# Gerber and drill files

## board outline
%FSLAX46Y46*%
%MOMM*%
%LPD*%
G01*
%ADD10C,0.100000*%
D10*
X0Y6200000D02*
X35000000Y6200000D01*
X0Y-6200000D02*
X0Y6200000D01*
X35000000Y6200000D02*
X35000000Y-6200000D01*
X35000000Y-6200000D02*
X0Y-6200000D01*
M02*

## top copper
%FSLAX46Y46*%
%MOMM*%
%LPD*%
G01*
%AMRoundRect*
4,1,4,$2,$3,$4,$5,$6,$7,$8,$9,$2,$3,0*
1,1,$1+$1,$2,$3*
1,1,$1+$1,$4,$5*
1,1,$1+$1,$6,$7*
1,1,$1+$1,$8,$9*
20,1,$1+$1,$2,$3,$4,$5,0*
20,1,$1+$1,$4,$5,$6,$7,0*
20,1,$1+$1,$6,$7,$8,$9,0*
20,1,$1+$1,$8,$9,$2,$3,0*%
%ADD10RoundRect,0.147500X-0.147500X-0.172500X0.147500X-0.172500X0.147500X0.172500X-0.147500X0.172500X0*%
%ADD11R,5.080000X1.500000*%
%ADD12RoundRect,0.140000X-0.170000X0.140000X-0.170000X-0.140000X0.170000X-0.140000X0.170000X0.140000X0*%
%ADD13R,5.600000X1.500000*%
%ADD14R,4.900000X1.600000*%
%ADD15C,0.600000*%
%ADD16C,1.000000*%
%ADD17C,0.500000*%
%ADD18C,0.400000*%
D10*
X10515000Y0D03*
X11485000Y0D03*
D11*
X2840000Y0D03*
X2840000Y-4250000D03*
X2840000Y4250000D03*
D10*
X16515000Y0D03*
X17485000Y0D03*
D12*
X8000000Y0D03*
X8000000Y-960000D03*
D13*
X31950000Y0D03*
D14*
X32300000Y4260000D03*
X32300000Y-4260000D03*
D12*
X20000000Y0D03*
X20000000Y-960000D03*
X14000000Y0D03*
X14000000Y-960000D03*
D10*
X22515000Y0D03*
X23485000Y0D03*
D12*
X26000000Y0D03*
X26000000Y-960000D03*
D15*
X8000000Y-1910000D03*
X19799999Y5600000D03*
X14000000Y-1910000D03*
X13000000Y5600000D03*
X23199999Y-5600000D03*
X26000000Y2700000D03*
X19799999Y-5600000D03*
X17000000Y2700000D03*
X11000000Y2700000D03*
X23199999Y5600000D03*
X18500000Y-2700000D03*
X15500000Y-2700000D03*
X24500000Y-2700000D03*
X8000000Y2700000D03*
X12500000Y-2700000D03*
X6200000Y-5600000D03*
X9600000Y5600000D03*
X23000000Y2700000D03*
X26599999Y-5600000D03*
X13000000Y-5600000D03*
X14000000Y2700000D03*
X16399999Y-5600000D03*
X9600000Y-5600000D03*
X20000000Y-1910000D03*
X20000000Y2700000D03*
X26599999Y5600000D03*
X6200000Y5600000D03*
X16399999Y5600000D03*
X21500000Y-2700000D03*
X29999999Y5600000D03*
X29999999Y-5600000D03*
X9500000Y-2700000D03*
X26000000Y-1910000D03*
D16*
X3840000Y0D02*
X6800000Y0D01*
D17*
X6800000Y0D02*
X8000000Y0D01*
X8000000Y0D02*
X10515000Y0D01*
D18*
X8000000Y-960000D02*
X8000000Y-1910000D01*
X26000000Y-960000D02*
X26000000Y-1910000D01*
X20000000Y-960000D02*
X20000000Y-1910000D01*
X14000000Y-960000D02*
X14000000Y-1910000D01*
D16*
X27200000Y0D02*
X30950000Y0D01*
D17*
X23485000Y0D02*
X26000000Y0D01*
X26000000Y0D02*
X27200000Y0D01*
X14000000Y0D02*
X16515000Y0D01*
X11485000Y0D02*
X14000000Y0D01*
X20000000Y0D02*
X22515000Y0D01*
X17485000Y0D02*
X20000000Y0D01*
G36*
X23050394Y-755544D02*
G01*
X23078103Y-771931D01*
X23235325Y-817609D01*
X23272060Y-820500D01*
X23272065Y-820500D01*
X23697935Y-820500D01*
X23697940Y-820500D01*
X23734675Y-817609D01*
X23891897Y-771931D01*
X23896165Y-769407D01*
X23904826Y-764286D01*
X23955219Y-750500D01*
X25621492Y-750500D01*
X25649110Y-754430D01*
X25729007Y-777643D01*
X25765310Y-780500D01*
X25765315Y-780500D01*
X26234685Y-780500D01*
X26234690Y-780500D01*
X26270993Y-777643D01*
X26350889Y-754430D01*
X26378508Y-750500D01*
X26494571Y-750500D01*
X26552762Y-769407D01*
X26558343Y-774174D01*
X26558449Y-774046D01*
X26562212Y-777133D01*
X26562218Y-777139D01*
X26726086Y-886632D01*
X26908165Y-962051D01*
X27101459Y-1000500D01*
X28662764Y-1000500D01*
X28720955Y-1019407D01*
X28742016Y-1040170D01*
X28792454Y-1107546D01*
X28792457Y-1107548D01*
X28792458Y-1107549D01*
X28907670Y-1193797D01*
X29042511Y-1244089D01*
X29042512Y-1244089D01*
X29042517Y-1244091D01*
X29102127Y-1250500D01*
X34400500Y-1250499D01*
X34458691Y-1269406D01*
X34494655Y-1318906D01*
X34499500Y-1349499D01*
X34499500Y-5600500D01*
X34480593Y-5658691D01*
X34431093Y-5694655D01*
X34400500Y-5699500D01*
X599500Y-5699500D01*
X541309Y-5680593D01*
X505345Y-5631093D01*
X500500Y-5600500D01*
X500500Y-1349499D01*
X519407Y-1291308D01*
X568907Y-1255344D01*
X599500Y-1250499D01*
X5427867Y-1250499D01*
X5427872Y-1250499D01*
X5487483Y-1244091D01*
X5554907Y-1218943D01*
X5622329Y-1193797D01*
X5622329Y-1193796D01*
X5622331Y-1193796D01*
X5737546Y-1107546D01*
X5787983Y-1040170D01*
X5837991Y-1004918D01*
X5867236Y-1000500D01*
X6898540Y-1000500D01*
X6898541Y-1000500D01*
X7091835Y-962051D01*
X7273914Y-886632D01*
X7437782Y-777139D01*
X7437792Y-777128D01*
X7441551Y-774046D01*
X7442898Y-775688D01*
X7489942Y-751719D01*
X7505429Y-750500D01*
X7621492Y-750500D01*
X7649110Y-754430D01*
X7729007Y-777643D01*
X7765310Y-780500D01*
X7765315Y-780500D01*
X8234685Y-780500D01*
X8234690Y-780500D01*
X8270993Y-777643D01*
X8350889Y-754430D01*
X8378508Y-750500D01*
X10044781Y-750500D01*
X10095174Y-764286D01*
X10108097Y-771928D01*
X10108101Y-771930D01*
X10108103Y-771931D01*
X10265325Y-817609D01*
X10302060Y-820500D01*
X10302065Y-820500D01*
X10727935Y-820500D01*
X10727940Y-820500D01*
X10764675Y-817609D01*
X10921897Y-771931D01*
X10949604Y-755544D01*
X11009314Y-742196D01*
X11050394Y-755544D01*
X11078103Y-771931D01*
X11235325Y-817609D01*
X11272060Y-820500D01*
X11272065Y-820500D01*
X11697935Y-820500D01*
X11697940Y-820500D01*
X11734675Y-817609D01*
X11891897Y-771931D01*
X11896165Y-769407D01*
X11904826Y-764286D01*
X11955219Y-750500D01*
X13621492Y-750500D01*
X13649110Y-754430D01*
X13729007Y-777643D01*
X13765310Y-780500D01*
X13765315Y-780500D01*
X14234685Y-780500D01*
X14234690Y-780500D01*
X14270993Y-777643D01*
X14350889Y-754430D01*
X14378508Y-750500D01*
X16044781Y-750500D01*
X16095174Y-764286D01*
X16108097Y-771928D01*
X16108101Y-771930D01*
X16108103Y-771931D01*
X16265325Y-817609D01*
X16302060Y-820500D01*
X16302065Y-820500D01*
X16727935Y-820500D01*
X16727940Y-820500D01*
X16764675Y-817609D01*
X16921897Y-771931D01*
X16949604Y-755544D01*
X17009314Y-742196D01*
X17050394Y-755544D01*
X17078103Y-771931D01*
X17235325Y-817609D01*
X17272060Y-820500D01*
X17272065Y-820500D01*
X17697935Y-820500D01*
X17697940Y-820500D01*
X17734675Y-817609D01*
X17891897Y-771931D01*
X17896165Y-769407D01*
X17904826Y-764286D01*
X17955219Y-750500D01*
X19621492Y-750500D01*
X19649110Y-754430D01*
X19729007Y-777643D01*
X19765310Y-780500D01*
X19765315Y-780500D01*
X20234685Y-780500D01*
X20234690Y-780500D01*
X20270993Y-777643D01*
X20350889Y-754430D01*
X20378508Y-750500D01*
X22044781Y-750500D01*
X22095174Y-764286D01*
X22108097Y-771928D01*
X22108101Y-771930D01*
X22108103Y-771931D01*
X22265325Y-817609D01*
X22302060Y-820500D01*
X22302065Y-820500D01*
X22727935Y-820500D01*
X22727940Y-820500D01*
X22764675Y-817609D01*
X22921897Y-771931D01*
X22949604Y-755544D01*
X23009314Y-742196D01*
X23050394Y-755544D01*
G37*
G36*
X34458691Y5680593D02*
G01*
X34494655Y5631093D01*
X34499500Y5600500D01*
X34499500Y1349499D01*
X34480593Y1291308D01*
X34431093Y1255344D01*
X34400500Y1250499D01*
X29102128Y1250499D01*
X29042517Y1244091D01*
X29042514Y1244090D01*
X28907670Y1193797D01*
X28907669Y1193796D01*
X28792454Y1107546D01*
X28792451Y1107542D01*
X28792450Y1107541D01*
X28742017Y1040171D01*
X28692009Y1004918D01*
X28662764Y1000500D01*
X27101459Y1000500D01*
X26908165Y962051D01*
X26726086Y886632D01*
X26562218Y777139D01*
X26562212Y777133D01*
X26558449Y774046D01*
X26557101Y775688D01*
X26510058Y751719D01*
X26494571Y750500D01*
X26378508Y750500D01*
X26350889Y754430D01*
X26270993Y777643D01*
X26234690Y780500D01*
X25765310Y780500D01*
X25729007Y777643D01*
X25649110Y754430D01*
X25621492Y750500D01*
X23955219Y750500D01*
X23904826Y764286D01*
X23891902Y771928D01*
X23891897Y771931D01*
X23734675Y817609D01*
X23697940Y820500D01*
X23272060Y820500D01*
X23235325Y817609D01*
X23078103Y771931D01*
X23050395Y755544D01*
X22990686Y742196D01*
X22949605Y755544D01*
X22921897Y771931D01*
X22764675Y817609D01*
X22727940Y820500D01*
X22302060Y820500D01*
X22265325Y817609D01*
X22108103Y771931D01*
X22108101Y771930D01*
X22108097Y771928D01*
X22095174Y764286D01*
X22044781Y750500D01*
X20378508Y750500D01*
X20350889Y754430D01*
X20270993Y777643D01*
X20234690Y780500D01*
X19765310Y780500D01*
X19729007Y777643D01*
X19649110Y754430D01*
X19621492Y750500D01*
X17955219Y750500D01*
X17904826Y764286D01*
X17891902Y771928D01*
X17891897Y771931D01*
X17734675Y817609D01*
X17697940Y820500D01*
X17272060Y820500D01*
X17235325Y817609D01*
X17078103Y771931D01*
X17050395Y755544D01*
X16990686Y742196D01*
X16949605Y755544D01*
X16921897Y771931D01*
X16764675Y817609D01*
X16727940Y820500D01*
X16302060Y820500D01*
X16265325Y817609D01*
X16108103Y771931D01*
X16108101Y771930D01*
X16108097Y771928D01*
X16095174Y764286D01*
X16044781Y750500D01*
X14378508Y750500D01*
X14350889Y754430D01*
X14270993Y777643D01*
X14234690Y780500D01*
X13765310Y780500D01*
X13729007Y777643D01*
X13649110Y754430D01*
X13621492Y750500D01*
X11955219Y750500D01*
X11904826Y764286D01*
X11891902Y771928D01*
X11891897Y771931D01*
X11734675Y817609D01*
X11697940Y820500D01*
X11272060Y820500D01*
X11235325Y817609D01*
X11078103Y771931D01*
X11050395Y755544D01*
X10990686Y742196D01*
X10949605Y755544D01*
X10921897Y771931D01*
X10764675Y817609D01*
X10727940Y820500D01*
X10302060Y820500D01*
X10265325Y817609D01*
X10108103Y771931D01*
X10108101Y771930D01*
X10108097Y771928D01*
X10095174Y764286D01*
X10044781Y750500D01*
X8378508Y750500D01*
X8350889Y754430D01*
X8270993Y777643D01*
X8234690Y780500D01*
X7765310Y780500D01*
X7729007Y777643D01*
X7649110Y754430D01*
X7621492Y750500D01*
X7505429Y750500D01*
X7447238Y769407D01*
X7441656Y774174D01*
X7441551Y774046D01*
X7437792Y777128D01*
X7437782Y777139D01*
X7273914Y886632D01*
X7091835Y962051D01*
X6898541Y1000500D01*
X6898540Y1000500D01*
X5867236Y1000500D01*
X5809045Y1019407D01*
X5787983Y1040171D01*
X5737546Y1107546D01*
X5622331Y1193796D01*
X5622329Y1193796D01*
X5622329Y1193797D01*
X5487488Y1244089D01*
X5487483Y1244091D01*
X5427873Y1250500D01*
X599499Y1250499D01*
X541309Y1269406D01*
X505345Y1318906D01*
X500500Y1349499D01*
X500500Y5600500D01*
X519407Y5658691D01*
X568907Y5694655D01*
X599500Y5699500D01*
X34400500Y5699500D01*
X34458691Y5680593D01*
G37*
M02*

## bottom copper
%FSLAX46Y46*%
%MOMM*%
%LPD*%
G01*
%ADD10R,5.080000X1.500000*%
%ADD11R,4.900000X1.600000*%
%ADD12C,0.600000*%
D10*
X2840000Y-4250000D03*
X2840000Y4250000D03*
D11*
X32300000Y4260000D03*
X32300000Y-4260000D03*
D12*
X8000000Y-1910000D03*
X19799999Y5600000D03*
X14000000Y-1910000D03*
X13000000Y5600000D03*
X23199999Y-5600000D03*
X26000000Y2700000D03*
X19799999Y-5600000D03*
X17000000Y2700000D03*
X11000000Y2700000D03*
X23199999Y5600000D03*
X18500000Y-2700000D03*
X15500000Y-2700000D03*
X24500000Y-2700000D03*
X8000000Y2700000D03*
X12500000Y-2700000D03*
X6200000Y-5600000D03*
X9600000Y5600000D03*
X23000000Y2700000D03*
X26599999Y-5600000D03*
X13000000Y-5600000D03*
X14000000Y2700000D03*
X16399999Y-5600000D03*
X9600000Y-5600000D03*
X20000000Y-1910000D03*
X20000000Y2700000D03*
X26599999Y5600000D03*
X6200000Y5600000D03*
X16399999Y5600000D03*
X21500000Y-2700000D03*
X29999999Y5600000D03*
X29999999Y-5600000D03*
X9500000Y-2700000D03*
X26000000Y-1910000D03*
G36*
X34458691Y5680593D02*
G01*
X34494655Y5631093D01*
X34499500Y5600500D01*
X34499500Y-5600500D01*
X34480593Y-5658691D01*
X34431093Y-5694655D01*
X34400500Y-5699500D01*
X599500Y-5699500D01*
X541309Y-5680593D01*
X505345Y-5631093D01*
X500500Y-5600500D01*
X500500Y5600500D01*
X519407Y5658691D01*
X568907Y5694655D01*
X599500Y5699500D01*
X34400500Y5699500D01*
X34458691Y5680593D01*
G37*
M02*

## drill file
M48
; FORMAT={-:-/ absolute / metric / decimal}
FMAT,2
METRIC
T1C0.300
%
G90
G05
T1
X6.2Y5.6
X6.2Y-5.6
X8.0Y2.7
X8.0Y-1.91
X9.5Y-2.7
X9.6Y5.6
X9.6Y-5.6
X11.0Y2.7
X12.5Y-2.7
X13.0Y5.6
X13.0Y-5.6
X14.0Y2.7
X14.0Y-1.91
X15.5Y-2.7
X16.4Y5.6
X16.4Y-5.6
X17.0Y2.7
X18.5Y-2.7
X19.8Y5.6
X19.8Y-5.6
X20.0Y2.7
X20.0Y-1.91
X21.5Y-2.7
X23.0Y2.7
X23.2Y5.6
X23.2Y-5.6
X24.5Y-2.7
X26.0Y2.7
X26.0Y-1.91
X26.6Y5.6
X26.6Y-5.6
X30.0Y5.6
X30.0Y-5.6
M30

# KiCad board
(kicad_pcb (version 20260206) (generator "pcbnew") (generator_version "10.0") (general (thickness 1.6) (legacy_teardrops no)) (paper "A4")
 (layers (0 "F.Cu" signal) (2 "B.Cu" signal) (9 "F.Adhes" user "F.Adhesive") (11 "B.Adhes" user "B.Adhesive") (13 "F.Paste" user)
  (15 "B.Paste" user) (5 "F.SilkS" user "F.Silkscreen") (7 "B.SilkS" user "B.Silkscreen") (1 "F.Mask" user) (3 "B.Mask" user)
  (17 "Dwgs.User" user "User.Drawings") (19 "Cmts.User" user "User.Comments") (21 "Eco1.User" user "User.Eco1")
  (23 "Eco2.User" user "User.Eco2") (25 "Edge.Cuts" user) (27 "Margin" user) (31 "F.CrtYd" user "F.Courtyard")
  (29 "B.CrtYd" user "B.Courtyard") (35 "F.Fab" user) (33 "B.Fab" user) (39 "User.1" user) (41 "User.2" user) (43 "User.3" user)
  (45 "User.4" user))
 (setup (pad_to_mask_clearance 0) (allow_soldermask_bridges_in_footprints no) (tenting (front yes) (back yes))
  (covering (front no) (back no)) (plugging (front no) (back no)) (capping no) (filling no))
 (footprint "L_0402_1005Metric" (layer "F.Cu") (at 11 0)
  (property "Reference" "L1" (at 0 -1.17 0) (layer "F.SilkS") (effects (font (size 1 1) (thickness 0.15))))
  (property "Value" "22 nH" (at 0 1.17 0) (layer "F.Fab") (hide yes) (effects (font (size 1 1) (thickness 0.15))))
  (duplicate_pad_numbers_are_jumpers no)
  (pad "1" smd roundrect (at -0.485 0) (size 0.59 0.64) (layers "F.Cu" "F.Mask" "F.Paste") (roundrect_rratio 0.25) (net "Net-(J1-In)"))
  (pad "2" smd roundrect (at 0.485 0) (size 0.59 0.64) (layers "F.Cu" "F.Mask" "F.Paste") (roundrect_rratio 0.25) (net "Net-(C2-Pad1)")))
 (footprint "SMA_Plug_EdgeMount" (layer "F.Cu") (at 2.84 0 180)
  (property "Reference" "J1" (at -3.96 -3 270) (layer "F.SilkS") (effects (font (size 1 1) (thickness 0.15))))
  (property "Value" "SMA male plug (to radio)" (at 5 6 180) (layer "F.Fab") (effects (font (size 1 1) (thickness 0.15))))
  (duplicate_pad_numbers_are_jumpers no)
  (pad "1" smd rect (at 0 0 270) (size 1.5 5.08) (layers "F.Cu" "F.Mask" "F.Paste") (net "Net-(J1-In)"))
  (pad "2" smd rect (at 0 -4.25 270) (size 1.5 5.08) (layers "F.Cu" "F.Mask" "F.Paste") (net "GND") (zone_connect 2))
  (pad "2" smd rect (at 0 -4.25 270) (size 1.5 5.08) (layers "B.Cu" "B.Mask" "B.Paste") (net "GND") (zone_connect 2))
  (pad "2" smd rect (at 0 4.25 270) (size 1.5 5.08) (layers "F.Cu" "F.Mask" "F.Paste") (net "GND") (zone_connect 2))
  (pad "2" smd rect (at 0 4.25 270) (size 1.5 5.08) (layers "B.Cu" "B.Mask" "B.Paste") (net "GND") (zone_connect 2)))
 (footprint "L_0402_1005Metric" (layer "F.Cu") (at 17 0)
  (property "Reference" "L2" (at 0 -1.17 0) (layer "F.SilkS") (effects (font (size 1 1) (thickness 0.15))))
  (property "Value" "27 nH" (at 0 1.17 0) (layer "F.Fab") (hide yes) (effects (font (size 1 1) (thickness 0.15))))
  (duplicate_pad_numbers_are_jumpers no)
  (pad "1" smd roundrect (at -0.485 0) (size 0.59 0.64) (layers "F.Cu" "F.Mask" "F.Paste") (roundrect_rratio 0.25) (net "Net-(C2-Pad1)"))
  (pad "2" smd roundrect (at 0.485 0) (size 0.59 0.64) (layers "F.Cu" "F.Mask" "F.Paste") (roundrect_rratio 0.25) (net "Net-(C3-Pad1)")))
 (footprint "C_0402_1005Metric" (layer "F.Cu") (at 8 0.48 -90)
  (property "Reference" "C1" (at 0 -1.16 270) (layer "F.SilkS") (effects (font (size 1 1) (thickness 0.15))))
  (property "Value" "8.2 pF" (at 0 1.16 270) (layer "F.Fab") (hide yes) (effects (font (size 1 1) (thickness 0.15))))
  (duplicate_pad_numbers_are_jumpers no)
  (pad "1" smd roundrect (at -0.48 0 270) (size 0.56 0.62) (layers "F.Cu" "F.Mask" "F.Paste") (roundrect_rratio 0.25) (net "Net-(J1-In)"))
  (pad "2" smd roundrect (at 0.48 0 270) (size 0.56 0.62) (layers "F.Cu" "F.Mask" "F.Paste") (roundrect_rratio 0.25) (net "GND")
   (zone_connect 2)))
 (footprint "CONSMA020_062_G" (layer "F.Cu") (at 34.75 0)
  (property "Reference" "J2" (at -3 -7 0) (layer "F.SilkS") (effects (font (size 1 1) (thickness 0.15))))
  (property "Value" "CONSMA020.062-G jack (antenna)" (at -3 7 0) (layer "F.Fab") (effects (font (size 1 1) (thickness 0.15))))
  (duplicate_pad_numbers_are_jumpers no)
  (pad "1" smd rect (at -2.8 0) (size 5.6 1.5) (layers "F.Cu" "F.Mask" "F.Paste") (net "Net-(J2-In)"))
  (pad "2" smd rect (at -2.45 -4.26) (size 4.9 1.6) (layers "F.Cu" "F.Mask" "F.Paste") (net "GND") (zone_connect 2))
  (pad "2" smd rect (at -2.45 -4.26) (size 4.9 1.6) (layers "B.Cu" "B.Mask" "B.Paste") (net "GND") (zone_connect 2))
  (pad "2" smd rect (at -2.45 4.26) (size 4.9 1.6) (layers "F.Cu" "F.Mask" "F.Paste") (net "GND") (zone_connect 2))
  (pad "2" smd rect (at -2.45 4.26) (size 4.9 1.6) (layers "B.Cu" "B.Mask" "B.Paste") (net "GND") (zone_connect 2)))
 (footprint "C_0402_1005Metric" (layer "F.Cu") (at 20 0.48 -90)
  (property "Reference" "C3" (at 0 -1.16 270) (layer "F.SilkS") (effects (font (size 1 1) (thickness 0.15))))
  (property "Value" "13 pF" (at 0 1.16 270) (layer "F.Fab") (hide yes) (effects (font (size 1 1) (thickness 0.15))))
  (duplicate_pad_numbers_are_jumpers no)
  (pad "1" smd roundrect (at -0.48 0 270) (size 0.56 0.62) (layers "F.Cu" "F.Mask" "F.Paste") (roundrect_rratio 0.25) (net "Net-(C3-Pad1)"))
  (pad "2" smd roundrect (at 0.48 0 270) (size 0.56 0.62) (layers "F.Cu" "F.Mask" "F.Paste") (roundrect_rratio 0.25) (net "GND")
   (zone_connect 2)))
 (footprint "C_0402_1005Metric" (layer "F.Cu") (at 14 0.48 -90)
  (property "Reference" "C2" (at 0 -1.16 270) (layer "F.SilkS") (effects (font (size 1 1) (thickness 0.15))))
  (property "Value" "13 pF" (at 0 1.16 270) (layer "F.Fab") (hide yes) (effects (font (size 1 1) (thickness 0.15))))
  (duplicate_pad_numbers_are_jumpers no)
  (pad "1" smd roundrect (at -0.48 0 270) (size 0.56 0.62) (layers "F.Cu" "F.Mask" "F.Paste") (roundrect_rratio 0.25) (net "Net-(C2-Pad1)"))
  (pad "2" smd roundrect (at 0.48 0 270) (size 0.56 0.62) (layers "F.Cu" "F.Mask" "F.Paste") (roundrect_rratio 0.25) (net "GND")
   (zone_connect 2)))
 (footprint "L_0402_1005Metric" (layer "F.Cu") (at 23 0)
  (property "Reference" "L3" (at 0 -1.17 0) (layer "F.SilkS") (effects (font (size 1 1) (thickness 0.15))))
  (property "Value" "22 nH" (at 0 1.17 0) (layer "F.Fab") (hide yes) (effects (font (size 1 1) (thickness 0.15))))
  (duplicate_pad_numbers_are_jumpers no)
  (pad "1" smd roundrect (at -0.485 0) (size 0.59 0.64) (layers "F.Cu" "F.Mask" "F.Paste") (roundrect_rratio 0.25) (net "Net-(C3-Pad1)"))
  (pad "2" smd roundrect (at 0.485 0) (size 0.59 0.64) (layers "F.Cu" "F.Mask" "F.Paste") (roundrect_rratio 0.25) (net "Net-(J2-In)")))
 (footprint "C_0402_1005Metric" (layer "F.Cu") (at 26 0.48 -90)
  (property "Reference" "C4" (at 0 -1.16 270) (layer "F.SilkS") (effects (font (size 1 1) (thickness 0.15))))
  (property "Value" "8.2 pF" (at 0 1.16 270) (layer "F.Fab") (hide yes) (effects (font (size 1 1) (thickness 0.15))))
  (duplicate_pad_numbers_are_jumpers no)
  (pad "1" smd roundrect (at -0.48 0 270) (size 0.56 0.62) (layers "F.Cu" "F.Mask" "F.Paste") (roundrect_rratio 0.25) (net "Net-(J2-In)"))
  (pad "2" smd roundrect (at 0.48 0 270) (size 0.56 0.62) (layers "F.Cu" "F.Mask" "F.Paste") (roundrect_rratio 0.25) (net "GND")
   (zone_connect 2)))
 (gr_line (start 0 -6.2) (end 35 -6.2) (stroke (width 0.1) (type default)) (layer "Edge.Cuts"))
 (gr_line (start 0 6.2) (end 0 -6.2) (stroke (width 0.1) (type default)) (layer "Edge.Cuts"))
 (gr_line (start 35 -6.2) (end 35 6.2) (stroke (width 0.1) (type default)) (layer "Edge.Cuts"))
 (gr_line (start 35 6.2) (end 0 6.2) (stroke (width 0.1) (type default)) (layer "Edge.Cuts"))
 (segment (start 3.84 0) (end 6.8 0) (width 1) (layer "F.Cu") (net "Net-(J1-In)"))
 (segment (start 6.8 0) (end 8 0) (width 0.5) (layer "F.Cu") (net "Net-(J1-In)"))
 (segment (start 8 0) (end 10.515 0) (width 0.5) (layer "F.Cu") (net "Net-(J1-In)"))
 (segment (start 8 0.96) (end 8 1.91) (width 0.4) (layer "F.Cu") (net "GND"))
 (segment (start 26 0.96) (end 26 1.91) (width 0.4) (layer "F.Cu") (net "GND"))
 (segment (start 20 0.96) (end 20 1.91) (width 0.4) (layer "F.Cu") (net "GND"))
 (segment (start 14 0.96) (end 14 1.91) (width 0.4) (layer "F.Cu") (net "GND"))
 (via (at 8 1.91) (size 0.6) (drill 0.3) (layers "F.Cu" "B.Cu") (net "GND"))
 (via (at 19.799999 -5.6) (size 0.6) (drill 0.3) (layers "F.Cu" "B.Cu") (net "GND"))
 (via (at 14 1.91) (size 0.6) (drill 0.3) (layers "F.Cu" "B.Cu") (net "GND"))
 (via (at 13 -5.6) (size 0.6) (drill 0.3) (layers "F.Cu" "B.Cu") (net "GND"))
 (via (at 23.199999 5.6) (size 0.6) (drill 0.3) (layers "F.Cu" "B.Cu") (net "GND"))
 (via (at 26 -2.7) (size 0.6) (drill 0.3) (layers "F.Cu" "B.Cu") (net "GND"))
 (via (at 19.799999 5.6) (size 0.6) (drill 0.3) (layers "F.Cu" "B.Cu") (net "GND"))
 (via (at 17 -2.7) (size 0.6) (drill 0.3) (layers "F.Cu" "B.Cu") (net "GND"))
 (via (at 11 -2.7) (size 0.6) (drill 0.3) (layers "F.Cu" "B.Cu") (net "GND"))
 (via (at 23.199999 -5.6) (size 0.6) (drill 0.3) (layers "F.Cu" "B.Cu") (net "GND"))
 (via (at 18.5 2.7) (size 0.6) (drill 0.3) (layers "F.Cu" "B.Cu") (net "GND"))
 (via (at 15.5 2.7) (size 0.6) (drill 0.3) (layers "F.Cu" "B.Cu") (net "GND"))
 (via (at 24.5 2.7) (size 0.6) (drill 0.3) (layers "F.Cu" "B.Cu") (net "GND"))
 (via (at 8 -2.7) (size 0.6) (drill 0.3) (layers "F.Cu" "B.Cu") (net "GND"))
 (via (at 12.5 2.7) (size 0.6) (drill 0.3) (layers "F.Cu" "B.Cu") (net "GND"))
 (via (at 6.2 5.6) (size 0.6) (drill 0.3) (layers "F.Cu" "B.Cu") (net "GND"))
 (via (at 9.6 -5.6) (size 0.6) (drill 0.3) (layers "F.Cu" "B.Cu") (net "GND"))
 (via (at 23 -2.7) (size 0.6) (drill 0.3) (layers "F.Cu" "B.Cu") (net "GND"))
 (via (at 26.599999 5.6) (size 0.6) (drill 0.3) (layers "F.Cu" "B.Cu") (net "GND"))
 (via (at 13 5.6) (size 0.6) (drill 0.3) (layers "F.Cu" "B.Cu") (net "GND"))
 (via (at 14 -2.7) (size 0.6) (drill 0.3) (layers "F.Cu" "B.Cu") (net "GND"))
 (via (at 16.399999 5.6) (size 0.6) (drill 0.3) (layers "F.Cu" "B.Cu") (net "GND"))
 (via (at 9.6 5.6) (size 0.6) (drill 0.3) (layers "F.Cu" "B.Cu") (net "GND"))
 (via (at 20 1.91) (size 0.6) (drill 0.3) (layers "F.Cu" "B.Cu") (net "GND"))
 (via (at 20 -2.7) (size 0.6) (drill 0.3) (layers "F.Cu" "B.Cu") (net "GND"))
 (via (at 26.599999 -5.6) (size 0.6) (drill 0.3) (layers "F.Cu" "B.Cu") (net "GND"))
 (via (at 6.2 -5.6) (size 0.6) (drill 0.3) (layers "F.Cu" "B.Cu") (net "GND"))
 (via (at 16.399999 -5.6) (size 0.6) (drill 0.3) (layers "F.Cu" "B.Cu") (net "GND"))
 (via (at 21.5 2.7) (size 0.6) (drill 0.3) (layers "F.Cu" "B.Cu") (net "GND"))
 (via (at 29.999999 -5.6) (size 0.6) (drill 0.3) (layers "F.Cu" "B.Cu") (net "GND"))
 (via (at 29.999999 5.6) (size 0.6) (drill 0.3) (layers "F.Cu" "B.Cu") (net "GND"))
 (via (at 9.5 2.7) (size 0.6) (drill 0.3) (layers "F.Cu" "B.Cu") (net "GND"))
 (via (at 26 1.91) (size 0.6) (drill 0.3) (layers "F.Cu" "B.Cu") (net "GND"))
 (segment (start 27.2 0) (end 30.95 0) (width 1) (layer "F.Cu") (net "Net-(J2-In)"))
 (segment (start 23.485 0) (end 26 0) (width 0.5) (layer "F.Cu") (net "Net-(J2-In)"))
 (segment (start 26 0) (end 27.2 0) (width 0.5) (layer "F.Cu") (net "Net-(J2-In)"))
 (segment (start 14 0) (end 16.515 0) (width 0.5) (layer "F.Cu") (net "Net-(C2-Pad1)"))
 (segment (start 11.485 0) (end 14 0) (width 0.5) (layer "F.Cu") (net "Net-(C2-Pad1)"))
 (segment (start 20 0) (end 22.515 0) (width 0.5) (layer "F.Cu") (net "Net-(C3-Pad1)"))
 (segment (start 17.485 0) (end 20 0) (width 0.5) (layer "F.Cu") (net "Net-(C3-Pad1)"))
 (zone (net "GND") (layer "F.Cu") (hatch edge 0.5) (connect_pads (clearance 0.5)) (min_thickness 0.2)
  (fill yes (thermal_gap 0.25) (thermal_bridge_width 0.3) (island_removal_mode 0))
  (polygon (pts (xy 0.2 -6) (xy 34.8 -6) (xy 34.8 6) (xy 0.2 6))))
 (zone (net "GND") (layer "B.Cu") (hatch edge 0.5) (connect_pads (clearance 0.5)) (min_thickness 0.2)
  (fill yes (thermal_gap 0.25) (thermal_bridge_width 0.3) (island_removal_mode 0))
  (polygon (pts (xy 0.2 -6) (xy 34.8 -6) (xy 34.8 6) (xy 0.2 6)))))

